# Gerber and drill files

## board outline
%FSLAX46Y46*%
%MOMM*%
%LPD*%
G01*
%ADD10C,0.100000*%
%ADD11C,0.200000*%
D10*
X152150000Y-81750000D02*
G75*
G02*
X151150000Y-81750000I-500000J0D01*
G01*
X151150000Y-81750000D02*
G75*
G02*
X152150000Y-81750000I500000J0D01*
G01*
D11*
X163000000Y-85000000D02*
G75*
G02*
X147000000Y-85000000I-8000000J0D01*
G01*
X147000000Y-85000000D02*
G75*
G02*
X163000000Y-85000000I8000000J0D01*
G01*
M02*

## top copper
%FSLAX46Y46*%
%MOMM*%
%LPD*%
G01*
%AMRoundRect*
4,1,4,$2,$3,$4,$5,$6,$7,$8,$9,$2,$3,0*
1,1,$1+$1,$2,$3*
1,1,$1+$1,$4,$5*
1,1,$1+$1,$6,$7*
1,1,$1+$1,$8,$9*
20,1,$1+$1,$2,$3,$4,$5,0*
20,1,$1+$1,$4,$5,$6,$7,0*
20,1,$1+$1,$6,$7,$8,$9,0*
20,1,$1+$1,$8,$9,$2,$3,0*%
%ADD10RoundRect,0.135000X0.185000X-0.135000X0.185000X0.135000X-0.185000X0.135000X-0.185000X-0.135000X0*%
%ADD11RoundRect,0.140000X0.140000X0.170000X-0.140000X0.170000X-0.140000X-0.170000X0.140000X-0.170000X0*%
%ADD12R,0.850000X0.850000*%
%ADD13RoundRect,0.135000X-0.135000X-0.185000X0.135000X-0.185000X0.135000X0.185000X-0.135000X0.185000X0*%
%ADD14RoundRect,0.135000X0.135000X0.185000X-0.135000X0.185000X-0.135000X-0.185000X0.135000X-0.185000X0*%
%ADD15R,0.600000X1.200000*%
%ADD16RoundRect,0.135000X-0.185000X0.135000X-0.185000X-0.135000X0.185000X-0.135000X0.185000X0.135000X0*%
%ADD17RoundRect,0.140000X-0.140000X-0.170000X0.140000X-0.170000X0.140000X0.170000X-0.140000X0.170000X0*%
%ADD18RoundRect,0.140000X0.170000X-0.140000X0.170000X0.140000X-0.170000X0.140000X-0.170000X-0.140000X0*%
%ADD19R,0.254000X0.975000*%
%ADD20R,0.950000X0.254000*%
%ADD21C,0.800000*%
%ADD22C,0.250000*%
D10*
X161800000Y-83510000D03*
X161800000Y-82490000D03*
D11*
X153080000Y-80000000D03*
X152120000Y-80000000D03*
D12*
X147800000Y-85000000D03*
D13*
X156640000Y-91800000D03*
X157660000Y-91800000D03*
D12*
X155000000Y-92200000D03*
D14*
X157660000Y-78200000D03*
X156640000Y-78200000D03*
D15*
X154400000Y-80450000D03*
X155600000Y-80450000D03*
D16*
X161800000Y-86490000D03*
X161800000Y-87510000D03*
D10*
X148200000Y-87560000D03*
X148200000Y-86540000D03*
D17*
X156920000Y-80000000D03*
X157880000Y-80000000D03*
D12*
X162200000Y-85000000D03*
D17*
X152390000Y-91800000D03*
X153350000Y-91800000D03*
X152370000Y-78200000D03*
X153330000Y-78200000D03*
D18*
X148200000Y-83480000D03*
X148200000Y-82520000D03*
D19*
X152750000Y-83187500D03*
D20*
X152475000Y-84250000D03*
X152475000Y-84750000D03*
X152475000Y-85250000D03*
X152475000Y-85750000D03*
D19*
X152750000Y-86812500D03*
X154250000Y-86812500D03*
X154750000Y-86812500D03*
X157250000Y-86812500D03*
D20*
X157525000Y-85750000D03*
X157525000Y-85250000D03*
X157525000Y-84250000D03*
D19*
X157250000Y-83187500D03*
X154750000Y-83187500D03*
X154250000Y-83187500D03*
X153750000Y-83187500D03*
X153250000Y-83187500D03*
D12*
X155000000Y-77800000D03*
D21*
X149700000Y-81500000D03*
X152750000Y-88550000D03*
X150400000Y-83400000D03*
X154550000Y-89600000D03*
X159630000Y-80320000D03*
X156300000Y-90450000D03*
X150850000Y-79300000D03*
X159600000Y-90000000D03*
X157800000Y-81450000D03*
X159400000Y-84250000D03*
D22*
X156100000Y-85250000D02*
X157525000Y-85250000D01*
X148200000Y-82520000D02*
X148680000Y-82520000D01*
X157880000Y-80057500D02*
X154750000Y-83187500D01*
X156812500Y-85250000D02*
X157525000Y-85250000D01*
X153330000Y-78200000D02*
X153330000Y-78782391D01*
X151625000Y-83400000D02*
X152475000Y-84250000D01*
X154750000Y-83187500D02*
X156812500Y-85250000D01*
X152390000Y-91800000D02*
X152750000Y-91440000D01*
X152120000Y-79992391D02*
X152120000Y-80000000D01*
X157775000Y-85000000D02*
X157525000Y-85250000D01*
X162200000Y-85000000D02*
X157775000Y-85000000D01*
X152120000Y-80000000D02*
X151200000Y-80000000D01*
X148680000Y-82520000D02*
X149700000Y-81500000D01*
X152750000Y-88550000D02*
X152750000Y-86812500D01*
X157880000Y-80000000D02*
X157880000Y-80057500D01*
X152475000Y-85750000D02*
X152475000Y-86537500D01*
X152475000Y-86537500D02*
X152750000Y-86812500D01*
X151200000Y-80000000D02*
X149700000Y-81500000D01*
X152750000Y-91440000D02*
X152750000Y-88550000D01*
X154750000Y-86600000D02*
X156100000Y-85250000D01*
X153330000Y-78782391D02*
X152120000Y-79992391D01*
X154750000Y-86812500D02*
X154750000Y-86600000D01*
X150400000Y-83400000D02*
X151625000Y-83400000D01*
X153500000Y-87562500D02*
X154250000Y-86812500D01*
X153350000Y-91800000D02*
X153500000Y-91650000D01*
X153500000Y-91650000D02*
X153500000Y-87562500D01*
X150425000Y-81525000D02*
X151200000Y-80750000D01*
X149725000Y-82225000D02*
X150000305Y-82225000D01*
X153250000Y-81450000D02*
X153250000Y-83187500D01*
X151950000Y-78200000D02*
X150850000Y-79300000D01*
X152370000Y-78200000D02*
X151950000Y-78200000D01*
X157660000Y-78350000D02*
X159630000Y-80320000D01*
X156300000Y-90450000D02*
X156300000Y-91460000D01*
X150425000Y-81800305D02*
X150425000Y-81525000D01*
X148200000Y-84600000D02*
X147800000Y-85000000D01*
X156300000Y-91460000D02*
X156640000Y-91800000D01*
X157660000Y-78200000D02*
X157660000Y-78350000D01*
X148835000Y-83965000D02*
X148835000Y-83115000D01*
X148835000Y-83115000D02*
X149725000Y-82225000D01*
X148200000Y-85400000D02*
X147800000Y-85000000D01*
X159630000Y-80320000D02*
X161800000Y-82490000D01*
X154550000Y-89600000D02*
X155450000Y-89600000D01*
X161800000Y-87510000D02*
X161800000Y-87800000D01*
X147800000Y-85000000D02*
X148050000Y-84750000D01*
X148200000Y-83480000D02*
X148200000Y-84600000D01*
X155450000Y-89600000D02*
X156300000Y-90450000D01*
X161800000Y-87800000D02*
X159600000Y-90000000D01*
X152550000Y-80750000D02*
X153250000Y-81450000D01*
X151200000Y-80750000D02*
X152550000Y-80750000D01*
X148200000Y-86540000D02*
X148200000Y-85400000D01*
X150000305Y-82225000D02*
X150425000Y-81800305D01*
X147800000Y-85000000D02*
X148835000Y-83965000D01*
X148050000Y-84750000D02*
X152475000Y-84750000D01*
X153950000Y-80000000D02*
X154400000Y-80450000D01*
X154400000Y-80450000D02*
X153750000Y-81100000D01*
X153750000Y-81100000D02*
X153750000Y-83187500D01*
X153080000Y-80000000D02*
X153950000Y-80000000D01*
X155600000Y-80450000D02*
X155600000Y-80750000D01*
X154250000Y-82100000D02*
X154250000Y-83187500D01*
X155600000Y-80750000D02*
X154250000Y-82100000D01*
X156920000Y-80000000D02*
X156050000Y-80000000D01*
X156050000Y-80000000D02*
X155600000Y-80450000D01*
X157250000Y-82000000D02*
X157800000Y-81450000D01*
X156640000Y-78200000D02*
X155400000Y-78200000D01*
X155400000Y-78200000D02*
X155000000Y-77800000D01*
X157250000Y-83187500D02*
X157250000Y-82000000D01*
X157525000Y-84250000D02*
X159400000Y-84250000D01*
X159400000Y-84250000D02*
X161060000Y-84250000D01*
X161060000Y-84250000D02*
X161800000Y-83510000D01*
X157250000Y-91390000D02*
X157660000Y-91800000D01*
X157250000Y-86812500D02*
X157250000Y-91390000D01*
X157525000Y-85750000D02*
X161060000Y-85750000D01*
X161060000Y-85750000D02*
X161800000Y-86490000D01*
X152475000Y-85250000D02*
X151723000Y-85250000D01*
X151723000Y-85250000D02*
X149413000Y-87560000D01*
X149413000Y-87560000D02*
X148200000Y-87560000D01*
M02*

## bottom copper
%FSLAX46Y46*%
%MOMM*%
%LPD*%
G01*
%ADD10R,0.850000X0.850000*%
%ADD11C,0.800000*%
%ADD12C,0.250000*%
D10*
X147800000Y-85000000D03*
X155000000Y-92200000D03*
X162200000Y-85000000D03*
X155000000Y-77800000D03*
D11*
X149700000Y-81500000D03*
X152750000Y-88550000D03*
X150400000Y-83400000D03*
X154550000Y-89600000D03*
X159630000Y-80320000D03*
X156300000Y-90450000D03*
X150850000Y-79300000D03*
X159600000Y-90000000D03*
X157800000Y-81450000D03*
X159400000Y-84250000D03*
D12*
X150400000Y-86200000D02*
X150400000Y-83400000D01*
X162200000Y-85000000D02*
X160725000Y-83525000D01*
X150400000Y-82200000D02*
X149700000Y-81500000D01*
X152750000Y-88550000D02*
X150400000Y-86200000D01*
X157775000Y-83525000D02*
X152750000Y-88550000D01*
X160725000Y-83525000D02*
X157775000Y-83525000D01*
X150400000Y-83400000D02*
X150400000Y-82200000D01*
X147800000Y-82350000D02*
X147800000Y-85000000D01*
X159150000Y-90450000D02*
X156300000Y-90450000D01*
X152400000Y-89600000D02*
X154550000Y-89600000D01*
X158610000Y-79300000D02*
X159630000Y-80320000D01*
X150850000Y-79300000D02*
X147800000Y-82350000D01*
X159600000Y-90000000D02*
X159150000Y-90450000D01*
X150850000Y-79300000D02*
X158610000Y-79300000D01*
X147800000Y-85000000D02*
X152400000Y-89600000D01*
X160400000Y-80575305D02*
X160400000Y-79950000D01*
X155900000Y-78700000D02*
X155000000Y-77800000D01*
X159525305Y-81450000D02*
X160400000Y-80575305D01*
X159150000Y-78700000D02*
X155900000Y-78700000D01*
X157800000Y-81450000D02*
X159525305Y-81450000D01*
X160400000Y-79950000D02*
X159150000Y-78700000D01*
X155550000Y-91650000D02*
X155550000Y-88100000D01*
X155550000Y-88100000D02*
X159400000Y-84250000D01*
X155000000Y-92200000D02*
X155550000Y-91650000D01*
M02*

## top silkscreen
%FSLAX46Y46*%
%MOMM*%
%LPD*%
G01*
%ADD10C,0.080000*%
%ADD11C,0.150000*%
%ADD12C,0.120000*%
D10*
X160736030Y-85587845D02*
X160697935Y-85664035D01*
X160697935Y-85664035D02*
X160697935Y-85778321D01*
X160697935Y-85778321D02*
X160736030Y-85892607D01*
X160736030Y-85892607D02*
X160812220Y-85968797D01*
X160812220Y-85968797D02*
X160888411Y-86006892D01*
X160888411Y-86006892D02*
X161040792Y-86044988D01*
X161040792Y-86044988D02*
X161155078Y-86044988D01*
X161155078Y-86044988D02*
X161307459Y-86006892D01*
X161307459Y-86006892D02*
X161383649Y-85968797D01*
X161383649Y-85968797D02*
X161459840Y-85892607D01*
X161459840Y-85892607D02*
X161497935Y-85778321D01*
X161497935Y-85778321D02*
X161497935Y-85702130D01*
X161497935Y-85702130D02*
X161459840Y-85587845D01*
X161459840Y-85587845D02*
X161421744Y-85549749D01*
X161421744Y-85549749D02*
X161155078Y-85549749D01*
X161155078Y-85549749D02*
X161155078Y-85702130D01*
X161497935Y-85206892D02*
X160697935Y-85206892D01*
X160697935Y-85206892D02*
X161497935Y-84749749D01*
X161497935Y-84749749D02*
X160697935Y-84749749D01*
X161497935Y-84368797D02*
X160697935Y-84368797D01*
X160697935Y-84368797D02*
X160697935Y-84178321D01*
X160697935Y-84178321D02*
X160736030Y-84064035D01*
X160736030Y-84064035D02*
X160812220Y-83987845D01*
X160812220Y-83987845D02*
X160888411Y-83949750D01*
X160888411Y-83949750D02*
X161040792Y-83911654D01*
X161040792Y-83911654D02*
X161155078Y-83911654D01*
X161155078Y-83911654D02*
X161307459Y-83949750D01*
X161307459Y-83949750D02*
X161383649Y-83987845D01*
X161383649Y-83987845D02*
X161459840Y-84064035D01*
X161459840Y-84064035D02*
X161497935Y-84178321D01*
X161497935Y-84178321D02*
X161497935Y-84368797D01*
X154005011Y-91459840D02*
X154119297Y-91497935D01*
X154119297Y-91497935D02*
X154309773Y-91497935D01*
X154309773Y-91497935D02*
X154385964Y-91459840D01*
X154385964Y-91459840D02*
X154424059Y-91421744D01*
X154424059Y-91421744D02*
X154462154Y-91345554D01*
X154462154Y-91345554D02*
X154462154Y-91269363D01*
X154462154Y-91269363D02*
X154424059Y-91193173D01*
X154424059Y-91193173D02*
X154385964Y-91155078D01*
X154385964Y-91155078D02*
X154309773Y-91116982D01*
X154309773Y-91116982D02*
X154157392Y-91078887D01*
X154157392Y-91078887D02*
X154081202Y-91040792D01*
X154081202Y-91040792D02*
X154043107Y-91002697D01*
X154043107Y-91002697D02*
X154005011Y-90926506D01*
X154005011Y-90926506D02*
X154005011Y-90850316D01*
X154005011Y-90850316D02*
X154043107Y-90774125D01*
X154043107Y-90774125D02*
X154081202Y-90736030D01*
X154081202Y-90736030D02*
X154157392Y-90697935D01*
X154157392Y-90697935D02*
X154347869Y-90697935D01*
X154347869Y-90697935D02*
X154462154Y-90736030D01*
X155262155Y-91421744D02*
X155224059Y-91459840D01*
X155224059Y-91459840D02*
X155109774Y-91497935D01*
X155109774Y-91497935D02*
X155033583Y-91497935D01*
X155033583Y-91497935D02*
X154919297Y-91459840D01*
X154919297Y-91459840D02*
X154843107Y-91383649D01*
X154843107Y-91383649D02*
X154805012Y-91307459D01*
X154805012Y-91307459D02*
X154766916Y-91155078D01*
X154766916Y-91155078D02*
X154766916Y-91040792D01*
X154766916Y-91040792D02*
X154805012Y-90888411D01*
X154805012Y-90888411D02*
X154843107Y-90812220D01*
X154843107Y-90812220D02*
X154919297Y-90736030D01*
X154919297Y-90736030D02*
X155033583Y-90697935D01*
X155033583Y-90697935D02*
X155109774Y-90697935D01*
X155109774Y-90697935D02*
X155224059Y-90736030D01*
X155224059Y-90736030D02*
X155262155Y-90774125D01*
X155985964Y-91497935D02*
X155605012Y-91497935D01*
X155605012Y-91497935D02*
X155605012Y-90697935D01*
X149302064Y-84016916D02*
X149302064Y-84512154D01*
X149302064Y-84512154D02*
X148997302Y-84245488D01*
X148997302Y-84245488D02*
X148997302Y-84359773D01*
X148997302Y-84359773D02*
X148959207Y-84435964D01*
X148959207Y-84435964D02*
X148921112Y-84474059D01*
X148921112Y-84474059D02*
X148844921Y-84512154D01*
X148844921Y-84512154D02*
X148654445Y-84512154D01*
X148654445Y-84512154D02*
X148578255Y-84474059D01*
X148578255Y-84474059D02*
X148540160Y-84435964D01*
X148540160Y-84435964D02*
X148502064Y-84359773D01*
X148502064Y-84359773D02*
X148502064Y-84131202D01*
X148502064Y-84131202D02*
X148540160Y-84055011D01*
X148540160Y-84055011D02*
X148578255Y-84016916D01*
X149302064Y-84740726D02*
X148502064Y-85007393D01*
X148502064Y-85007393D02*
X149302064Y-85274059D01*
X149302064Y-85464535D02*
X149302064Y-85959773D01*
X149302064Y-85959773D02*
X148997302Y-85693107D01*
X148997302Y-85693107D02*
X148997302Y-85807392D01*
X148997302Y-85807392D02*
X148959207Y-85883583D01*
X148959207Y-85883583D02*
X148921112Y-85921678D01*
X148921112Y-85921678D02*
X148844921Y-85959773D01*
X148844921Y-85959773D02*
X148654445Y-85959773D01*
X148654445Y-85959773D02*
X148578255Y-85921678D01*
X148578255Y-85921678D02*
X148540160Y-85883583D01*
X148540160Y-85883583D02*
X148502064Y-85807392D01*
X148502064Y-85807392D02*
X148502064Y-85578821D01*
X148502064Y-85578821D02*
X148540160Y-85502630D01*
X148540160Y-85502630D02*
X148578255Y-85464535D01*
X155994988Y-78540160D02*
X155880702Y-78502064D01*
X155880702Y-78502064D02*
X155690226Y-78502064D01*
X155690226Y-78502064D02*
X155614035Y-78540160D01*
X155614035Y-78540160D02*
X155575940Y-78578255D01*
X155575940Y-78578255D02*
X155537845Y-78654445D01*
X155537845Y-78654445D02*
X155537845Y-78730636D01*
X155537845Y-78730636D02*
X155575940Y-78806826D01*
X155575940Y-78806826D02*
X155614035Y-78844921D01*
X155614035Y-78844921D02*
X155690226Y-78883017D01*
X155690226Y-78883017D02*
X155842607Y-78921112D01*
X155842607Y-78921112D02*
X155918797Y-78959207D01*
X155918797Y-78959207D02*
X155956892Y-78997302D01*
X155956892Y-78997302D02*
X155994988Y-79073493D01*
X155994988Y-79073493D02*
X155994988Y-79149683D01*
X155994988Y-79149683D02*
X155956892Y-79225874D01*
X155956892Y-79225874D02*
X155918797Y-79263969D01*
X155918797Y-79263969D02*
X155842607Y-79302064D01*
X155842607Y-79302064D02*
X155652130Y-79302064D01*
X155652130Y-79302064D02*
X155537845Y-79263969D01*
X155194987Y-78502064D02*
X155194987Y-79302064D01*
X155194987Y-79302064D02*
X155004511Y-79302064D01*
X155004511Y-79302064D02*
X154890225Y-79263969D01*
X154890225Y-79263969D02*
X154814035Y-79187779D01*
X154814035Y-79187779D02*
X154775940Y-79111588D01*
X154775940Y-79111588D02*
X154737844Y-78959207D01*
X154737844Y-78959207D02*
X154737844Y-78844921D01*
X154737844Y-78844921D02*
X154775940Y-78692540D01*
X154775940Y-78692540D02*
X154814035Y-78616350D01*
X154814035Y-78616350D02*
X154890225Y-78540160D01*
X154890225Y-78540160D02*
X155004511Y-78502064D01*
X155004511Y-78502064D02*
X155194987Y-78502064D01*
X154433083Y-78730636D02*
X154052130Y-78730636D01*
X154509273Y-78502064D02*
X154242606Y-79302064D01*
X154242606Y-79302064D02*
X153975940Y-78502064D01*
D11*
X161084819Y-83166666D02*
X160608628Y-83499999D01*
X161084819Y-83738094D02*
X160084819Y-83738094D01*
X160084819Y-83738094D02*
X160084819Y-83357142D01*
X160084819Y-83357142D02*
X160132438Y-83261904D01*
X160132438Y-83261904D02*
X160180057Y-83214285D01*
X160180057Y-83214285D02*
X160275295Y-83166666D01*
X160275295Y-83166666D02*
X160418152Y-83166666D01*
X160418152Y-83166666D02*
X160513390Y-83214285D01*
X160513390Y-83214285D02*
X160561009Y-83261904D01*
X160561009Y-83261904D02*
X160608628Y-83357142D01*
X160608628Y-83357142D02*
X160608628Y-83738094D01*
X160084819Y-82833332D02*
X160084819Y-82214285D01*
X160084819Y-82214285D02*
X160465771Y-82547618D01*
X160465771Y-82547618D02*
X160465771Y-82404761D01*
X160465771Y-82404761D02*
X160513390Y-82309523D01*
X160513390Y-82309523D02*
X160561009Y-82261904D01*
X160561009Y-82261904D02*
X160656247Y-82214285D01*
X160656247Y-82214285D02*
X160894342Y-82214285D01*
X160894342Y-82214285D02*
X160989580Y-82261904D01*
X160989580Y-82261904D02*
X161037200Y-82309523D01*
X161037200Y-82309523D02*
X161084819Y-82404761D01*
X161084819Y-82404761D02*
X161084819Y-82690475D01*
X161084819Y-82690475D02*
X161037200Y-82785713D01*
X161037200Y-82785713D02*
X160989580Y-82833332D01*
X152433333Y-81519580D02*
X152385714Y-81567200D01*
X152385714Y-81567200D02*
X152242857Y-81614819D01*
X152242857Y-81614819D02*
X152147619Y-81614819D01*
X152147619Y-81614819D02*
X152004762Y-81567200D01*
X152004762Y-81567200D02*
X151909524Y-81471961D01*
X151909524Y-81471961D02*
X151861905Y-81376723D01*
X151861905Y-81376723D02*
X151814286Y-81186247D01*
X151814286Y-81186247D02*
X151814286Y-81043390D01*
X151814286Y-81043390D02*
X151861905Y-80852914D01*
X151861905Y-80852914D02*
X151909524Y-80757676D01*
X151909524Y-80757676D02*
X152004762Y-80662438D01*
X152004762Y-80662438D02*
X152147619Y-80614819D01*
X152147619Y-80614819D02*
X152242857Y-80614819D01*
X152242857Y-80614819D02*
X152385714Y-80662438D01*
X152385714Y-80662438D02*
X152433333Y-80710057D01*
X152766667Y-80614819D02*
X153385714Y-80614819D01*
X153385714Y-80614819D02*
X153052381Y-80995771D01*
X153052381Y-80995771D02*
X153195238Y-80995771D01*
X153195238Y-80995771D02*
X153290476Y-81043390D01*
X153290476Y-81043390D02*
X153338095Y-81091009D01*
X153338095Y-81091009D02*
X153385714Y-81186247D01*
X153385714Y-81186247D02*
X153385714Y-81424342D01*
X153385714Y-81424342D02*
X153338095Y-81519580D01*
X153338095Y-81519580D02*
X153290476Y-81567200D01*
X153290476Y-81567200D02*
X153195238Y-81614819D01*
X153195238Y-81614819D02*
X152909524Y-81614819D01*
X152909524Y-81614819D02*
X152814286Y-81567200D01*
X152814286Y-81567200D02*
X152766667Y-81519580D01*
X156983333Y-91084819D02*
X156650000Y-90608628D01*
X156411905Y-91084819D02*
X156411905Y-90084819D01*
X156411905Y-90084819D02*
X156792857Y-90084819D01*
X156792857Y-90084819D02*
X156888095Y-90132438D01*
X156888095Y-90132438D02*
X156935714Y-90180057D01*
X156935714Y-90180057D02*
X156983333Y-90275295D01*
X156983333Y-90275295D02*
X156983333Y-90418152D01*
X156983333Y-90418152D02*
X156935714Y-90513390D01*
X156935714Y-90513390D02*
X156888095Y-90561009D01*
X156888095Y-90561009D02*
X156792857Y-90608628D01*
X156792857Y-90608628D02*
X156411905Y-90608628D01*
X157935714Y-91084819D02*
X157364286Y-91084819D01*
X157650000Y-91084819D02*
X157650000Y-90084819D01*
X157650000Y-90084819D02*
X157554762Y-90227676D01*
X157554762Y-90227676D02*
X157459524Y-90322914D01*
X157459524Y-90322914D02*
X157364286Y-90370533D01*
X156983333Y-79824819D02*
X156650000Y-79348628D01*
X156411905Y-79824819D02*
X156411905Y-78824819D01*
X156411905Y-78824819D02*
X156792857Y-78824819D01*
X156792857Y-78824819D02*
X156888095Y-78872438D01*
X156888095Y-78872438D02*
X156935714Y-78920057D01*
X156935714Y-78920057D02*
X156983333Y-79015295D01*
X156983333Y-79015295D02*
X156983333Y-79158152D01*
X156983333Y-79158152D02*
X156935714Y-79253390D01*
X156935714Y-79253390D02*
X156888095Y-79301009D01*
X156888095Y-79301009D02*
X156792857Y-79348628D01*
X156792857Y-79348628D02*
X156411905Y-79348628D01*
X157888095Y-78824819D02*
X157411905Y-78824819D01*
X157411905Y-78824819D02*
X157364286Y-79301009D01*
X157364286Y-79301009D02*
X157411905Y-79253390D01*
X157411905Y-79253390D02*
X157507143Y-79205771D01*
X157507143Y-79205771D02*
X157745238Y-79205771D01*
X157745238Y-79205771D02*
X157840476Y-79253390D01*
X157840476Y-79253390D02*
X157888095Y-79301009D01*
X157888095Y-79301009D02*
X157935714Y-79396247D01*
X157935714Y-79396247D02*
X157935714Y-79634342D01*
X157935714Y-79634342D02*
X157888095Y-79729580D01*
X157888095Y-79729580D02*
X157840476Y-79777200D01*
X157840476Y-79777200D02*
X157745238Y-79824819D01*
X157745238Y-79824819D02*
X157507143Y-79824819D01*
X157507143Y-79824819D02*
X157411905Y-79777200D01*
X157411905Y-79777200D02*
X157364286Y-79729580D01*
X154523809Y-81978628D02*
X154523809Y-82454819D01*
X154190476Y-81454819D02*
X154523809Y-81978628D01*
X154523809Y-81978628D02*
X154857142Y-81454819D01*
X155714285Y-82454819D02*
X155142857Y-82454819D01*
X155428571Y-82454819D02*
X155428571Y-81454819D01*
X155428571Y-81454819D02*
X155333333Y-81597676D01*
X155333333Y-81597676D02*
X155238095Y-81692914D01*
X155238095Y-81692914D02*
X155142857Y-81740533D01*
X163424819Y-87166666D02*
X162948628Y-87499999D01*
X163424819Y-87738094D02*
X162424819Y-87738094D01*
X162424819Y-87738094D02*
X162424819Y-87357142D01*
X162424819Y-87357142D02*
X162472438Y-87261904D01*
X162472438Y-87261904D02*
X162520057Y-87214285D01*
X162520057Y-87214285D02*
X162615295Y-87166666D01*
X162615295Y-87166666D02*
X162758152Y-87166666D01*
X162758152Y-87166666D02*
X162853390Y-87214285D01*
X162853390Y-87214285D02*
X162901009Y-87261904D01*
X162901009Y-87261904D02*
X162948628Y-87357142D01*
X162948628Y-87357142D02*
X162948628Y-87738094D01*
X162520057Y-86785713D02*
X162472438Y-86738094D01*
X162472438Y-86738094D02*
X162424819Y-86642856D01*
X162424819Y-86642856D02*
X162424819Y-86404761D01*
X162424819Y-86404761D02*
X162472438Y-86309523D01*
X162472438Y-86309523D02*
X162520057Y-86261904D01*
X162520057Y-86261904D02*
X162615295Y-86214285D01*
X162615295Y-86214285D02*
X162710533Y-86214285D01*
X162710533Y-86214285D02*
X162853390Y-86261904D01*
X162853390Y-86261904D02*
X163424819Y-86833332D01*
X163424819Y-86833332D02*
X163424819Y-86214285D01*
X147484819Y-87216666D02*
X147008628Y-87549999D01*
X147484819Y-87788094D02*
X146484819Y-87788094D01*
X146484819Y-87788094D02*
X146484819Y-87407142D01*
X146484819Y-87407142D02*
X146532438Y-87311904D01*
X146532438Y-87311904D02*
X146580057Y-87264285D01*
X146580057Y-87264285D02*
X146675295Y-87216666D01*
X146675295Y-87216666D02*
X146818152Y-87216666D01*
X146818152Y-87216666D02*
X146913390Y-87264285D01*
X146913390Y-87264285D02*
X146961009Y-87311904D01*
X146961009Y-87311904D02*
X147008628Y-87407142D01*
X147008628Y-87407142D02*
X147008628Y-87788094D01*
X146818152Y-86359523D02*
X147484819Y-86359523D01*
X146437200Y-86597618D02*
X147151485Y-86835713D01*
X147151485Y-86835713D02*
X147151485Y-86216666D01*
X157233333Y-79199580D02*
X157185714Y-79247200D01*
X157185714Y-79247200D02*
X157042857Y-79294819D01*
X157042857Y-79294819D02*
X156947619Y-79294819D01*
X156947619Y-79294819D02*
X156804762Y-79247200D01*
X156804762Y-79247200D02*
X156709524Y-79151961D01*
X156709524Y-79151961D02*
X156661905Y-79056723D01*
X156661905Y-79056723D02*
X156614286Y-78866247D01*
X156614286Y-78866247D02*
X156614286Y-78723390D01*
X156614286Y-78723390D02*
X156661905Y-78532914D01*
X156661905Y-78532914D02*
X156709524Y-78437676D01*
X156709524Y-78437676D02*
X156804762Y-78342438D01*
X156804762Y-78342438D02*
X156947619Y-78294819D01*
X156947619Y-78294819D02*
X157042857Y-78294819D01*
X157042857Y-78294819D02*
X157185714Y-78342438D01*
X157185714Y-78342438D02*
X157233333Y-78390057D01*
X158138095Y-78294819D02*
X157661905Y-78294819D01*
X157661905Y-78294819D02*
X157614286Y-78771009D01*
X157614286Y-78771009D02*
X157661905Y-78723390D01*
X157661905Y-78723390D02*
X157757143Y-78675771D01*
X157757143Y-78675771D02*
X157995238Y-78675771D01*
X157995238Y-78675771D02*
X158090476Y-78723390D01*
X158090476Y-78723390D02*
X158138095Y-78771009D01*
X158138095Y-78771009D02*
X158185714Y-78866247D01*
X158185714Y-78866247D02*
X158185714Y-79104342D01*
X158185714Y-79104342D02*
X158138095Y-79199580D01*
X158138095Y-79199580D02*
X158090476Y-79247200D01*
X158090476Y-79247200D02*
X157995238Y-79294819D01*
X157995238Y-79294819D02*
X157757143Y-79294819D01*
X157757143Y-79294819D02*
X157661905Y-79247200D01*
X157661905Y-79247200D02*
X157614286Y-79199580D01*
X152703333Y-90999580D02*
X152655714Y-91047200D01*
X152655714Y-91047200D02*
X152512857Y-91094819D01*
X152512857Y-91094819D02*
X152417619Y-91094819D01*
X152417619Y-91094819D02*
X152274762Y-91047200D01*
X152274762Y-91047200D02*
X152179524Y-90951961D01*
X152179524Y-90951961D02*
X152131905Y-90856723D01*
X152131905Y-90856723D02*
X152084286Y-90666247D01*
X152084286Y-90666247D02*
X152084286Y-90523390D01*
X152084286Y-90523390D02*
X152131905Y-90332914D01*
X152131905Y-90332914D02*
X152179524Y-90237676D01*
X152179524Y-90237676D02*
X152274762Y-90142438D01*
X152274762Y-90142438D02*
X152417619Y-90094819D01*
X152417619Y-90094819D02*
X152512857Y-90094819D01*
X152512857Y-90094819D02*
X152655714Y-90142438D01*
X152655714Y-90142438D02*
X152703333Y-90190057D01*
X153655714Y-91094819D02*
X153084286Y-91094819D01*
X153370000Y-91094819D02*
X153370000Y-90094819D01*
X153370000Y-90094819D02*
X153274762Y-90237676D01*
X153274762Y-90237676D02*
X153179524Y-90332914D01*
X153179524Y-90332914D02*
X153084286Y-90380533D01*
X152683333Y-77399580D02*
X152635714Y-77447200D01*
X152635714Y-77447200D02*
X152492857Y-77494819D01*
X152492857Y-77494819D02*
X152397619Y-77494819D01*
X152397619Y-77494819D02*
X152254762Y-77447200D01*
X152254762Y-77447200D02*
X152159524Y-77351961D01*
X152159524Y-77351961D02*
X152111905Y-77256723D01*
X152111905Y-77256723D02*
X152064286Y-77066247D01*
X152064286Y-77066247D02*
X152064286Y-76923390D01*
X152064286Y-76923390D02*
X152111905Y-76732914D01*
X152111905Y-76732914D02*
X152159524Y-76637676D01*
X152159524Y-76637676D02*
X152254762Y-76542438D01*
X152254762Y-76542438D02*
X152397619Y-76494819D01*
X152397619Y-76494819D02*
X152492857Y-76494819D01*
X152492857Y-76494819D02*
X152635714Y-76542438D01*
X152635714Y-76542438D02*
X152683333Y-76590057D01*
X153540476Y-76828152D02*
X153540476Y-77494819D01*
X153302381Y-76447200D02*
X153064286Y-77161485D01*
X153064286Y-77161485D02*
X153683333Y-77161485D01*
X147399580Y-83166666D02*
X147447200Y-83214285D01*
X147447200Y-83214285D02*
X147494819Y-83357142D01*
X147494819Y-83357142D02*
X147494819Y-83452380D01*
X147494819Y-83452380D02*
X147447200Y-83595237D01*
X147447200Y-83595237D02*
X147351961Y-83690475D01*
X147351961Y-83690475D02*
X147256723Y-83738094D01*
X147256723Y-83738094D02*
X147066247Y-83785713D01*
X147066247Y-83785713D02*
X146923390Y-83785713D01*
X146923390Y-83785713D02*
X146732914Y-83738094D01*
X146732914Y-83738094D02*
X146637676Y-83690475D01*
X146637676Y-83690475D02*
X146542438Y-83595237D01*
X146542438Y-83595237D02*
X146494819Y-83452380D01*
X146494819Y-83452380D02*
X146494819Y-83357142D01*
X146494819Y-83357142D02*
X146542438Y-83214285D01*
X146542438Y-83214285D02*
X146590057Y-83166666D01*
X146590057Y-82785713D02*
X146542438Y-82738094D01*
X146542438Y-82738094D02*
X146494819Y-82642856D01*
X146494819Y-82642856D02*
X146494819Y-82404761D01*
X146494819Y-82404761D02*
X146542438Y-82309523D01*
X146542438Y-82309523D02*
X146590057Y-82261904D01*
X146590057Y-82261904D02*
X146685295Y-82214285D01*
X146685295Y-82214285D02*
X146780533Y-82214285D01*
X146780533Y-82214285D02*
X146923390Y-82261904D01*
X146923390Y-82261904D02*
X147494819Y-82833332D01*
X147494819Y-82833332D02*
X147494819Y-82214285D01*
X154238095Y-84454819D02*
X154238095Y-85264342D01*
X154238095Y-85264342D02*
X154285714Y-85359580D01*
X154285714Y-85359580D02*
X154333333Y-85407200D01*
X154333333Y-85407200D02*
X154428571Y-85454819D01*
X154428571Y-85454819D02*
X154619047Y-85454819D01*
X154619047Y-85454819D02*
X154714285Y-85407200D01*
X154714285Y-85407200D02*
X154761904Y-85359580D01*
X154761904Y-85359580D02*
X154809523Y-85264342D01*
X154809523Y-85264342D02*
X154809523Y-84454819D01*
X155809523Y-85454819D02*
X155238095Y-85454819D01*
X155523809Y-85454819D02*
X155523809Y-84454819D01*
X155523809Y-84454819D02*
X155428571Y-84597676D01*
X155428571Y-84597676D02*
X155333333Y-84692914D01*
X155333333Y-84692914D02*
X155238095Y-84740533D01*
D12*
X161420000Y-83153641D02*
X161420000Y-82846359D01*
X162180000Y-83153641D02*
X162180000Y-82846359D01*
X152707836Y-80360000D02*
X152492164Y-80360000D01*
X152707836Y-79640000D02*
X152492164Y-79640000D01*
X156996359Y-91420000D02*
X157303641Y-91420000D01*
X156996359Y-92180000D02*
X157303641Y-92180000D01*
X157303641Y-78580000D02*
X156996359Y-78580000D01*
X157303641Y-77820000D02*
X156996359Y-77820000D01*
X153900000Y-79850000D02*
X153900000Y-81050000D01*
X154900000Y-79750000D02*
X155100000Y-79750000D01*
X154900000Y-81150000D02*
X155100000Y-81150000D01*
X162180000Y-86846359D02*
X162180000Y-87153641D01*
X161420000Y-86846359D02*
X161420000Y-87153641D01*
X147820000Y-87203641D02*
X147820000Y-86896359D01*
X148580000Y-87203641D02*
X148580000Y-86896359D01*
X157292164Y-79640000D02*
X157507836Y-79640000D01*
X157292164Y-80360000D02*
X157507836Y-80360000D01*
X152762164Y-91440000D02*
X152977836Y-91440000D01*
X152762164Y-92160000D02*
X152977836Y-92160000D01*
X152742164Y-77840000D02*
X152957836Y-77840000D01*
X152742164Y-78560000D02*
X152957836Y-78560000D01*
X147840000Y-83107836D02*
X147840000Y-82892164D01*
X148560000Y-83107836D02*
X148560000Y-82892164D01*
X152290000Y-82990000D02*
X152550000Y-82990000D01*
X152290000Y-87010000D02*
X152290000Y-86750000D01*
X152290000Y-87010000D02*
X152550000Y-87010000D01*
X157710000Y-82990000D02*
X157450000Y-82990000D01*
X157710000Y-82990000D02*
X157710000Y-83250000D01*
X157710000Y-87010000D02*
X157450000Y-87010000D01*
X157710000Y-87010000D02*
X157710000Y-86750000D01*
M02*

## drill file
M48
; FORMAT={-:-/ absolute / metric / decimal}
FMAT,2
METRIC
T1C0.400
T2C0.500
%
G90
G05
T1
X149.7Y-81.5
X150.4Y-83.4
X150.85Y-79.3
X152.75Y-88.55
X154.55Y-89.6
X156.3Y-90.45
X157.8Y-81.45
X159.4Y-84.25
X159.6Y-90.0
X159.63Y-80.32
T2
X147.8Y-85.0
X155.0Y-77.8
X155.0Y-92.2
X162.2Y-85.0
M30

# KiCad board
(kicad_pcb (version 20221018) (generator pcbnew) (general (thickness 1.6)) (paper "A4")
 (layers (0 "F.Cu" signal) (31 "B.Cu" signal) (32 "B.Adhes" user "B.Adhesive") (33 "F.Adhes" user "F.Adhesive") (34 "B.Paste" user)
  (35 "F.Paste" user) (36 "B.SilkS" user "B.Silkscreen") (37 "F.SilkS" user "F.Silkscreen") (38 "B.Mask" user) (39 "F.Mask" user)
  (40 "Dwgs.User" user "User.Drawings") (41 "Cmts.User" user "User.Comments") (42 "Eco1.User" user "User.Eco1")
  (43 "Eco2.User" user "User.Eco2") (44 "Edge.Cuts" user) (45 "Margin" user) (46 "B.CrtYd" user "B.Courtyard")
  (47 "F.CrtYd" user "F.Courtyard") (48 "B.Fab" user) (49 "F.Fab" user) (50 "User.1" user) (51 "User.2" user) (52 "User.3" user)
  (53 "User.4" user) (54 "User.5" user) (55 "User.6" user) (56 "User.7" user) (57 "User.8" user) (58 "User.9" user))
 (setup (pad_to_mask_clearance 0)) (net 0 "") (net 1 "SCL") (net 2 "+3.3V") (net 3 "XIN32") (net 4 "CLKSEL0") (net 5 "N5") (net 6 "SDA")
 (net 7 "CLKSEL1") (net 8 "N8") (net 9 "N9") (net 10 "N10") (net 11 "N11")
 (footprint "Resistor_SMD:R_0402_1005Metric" (layer "F.Cu") (at 161.8 83 90)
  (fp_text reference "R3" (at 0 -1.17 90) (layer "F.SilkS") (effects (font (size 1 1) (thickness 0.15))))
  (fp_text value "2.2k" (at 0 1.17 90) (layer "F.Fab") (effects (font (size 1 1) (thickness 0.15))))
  (fp_line (start -0.153641 -0.38) (end 0.153641 -0.38) (stroke (width 0.12) (type solid)) (layer "F.SilkS"))
  (fp_line (start -0.153641 0.38) (end 0.153641 0.38) (stroke (width 0.12) (type solid)) (layer "F.SilkS"))
  (pad "1" smd roundrect (at -0.51 0 90) (size 0.54 0.64) (layers "F.Cu" "F.Paste" "F.Mask") (roundrect_rratio 0.25) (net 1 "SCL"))
  (pad "2" smd roundrect (at 0.51 0 90) (size 0.54 0.64) (layers "F.Cu" "F.Paste" "F.Mask") (roundrect_rratio 0.25) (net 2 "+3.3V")))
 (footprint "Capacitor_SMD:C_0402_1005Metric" (layer "F.Cu") (at 152.6 80 180)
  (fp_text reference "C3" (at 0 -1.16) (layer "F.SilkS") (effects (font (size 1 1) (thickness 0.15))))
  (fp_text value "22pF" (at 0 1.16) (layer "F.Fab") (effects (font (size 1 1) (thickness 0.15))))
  (fp_line (start -0.107836 -0.36) (end 0.107836 -0.36) (stroke (width 0.12) (type solid)) (layer "F.SilkS"))
  (fp_line (start -0.107836 0.36) (end 0.107836 0.36) (stroke (width 0.12) (type solid)) (layer "F.SilkS"))
  (pad "1" smd roundrect (at -0.48 0 180) (size 0.56 0.62) (layers "F.Cu" "F.Paste" "F.Mask") (roundrect_rratio 0.25) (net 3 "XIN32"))
  (pad "2" smd roundrect (at 0.48 0 180) (size 0.56 0.62) (layers "F.Cu" "F.Paste" "F.Mask") (roundrect_rratio 0.25) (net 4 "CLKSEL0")))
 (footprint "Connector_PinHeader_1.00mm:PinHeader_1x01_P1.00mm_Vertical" (layer "F.Cu") (at 147.8 85)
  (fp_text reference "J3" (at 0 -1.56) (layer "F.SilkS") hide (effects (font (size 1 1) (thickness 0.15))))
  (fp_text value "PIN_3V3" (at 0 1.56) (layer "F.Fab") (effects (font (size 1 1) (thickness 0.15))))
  (pad "1" thru_hole rect (at 0 0) (size 0.85 0.85) (drill 0.5) (layers "*.Cu" "*.Mask") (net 2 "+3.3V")))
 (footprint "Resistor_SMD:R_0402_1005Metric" (layer "F.Cu") (at 157.15 91.8)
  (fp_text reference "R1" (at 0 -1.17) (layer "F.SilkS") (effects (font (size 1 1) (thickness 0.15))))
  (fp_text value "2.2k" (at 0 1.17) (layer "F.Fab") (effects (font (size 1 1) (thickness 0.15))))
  (fp_line (start -0.153641 -0.38) (end 0.153641 -0.38) (stroke (width 0.12) (type solid)) (layer "F.SilkS"))
  (fp_line (start -0.153641 0.38) (end 0.153641 0.38) (stroke (width 0.12) (type solid)) (layer "F.SilkS"))
  (pad "1" smd roundrect (at -0.51 0) (size 0.54 0.64) (layers "F.Cu" "F.Paste" "F.Mask") (roundrect_rratio 0.25) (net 2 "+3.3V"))
  (pad "2" smd roundrect (at 0.51 0) (size 0.54 0.64) (layers "F.Cu" "F.Paste" "F.Mask") (roundrect_rratio 0.25) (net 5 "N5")))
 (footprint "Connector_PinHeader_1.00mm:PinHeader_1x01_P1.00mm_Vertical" (layer "F.Cu") (at 155 92.2)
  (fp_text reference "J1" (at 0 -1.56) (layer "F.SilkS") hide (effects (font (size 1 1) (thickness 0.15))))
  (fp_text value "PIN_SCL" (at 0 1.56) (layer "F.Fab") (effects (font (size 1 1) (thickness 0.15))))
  (pad "1" thru_hole rect (at 0 0) (size 0.85 0.85) (drill 0.5) (layers "*.Cu" "*.Mask") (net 1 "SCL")))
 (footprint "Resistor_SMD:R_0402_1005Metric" (layer "F.Cu") (at 157.15 78.2 180)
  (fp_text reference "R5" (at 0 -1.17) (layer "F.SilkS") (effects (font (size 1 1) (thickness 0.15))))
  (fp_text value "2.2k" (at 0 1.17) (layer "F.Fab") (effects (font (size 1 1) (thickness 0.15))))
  (fp_line (start -0.153641 -0.38) (end 0.153641 -0.38) (stroke (width 0.12) (type solid)) (layer "F.SilkS"))
  (fp_line (start -0.153641 0.38) (end 0.153641 0.38) (stroke (width 0.12) (type solid)) (layer "F.SilkS"))
  (pad "1" smd roundrect (at -0.51 0 180) (size 0.54 0.64) (layers "F.Cu" "F.Paste" "F.Mask") (roundrect_rratio 0.25) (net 2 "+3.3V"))
  (pad "2" smd roundrect (at 0.51 0 180) (size 0.54 0.64) (layers "F.Cu" "F.Paste" "F.Mask") (roundrect_rratio 0.25) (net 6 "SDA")))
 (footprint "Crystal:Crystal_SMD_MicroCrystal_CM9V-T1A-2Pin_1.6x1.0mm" (layer "F.Cu") (at 155 80.45)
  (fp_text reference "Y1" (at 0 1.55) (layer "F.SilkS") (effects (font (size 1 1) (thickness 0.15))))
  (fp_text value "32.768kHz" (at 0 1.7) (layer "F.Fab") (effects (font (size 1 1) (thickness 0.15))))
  (fp_line (start -1.1 -0.6) (end -1.1 0.6) (stroke (width 0.12) (type solid)) (layer "F.SilkS"))
  (fp_line (start -0.1 -0.7) (end 0.1 -0.7) (stroke (width 0.12) (type solid)) (layer "F.SilkS"))
  (fp_line (start -0.1 0.7) (end 0.1 0.7) (stroke (width 0.12) (type solid)) (layer "F.SilkS"))
  (pad "1" smd rect (at -0.6 0) (size 0.6 1.2) (layers "F.Cu" "F.Paste" "F.Mask") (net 3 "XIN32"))
  (pad "2" smd rect (at 0.6 0) (size 0.6 1.2) (layers "F.Cu" "F.Paste" "F.Mask") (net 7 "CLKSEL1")))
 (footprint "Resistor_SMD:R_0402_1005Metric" (layer "F.Cu") (at 161.8 87 -90)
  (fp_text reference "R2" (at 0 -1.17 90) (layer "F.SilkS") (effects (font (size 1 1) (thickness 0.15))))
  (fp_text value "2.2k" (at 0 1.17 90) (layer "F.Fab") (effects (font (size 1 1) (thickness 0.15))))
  (fp_line (start -0.153641 -0.38) (end 0.153641 -0.38) (stroke (width 0.12) (type solid)) (layer "F.SilkS"))
  (fp_line (start -0.153641 0.38) (end 0.153641 0.38) (stroke (width 0.12) (type solid)) (layer "F.SilkS"))
  (pad "1" smd roundrect (at -0.51 0 270) (size 0.54 0.64) (layers "F.Cu" "F.Paste" "F.Mask") (roundrect_rratio 0.25) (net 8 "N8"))
  (pad "2" smd roundrect (at 0.51 0 270) (size 0.54 0.64) (layers "F.Cu" "F.Paste" "F.Mask") (roundrect_rratio 0.25) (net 2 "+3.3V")))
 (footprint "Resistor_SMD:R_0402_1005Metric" (layer "F.Cu") (at 148.2 87.05 90)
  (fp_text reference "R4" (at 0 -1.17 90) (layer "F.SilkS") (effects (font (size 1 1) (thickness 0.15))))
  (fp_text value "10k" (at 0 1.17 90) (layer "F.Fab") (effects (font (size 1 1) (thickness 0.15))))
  (fp_line (start -0.153641 -0.38) (end 0.153641 -0.38) (stroke (width 0.12) (type solid)) (layer "F.SilkS"))
  (fp_line (start -0.153641 0.38) (end 0.153641 0.38) (stroke (width 0.12) (type solid)) (layer "F.SilkS"))
  (pad "1" smd roundrect (at -0.51 0 90) (size 0.54 0.64) (layers "F.Cu" "F.Paste" "F.Mask") (roundrect_rratio 0.25) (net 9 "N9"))
  (pad "2" smd roundrect (at 0.51 0 90) (size 0.54 0.64) (layers "F.Cu" "F.Paste" "F.Mask") (roundrect_rratio 0.25) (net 2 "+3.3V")))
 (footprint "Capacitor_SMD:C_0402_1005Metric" (layer "F.Cu") (at 157.4 80)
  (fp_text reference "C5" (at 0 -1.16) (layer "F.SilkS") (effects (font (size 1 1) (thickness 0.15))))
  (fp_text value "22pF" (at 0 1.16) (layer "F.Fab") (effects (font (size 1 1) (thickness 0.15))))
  (fp_line (start -0.107836 -0.36) (end 0.107836 -0.36) (stroke (width 0.12) (type solid)) (layer "F.SilkS"))
  (fp_line (start -0.107836 0.36) (end 0.107836 0.36) (stroke (width 0.12) (type solid)) (layer "F.SilkS"))
  (pad "1" smd roundrect (at -0.48 0) (size 0.56 0.62) (layers "F.Cu" "F.Paste" "F.Mask") (roundrect_rratio 0.25) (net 7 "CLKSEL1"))
  (pad "2" smd roundrect (at 0.48 0) (size 0.56 0.62) (layers "F.Cu" "F.Paste" "F.Mask") (roundrect_rratio 0.25) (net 4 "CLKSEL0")))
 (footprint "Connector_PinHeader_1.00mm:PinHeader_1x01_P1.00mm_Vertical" (layer "F.Cu") (at 162.2 85)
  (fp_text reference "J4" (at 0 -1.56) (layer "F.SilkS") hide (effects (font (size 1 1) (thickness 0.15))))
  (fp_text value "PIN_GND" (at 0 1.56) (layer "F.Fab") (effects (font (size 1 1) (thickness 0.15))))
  (pad "1" thru_hole rect (at 0 0) (size 0.85 0.85) (drill 0.5) (layers "*.Cu" "*.Mask") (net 4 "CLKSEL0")))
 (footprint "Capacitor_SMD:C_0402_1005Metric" (layer "F.Cu") (at 152.87 91.8)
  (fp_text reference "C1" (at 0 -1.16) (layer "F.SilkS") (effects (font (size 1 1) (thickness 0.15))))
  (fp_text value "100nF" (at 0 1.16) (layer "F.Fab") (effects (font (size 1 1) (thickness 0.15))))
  (fp_line (start -0.107836 -0.36) (end 0.107836 -0.36) (stroke (width 0.12) (type solid)) (layer "F.SilkS"))
  (fp_line (start -0.107836 0.36) (end 0.107836 0.36) (stroke (width 0.12) (type solid)) (layer "F.SilkS"))
  (pad "1" smd roundrect (at -0.48 0) (size 0.56 0.62) (layers "F.Cu" "F.Paste" "F.Mask") (roundrect_rratio 0.25) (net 4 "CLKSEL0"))
  (pad "2" smd roundrect (at 0.48 0) (size 0.56 0.62) (layers "F.Cu" "F.Paste" "F.Mask") (roundrect_rratio 0.25) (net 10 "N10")))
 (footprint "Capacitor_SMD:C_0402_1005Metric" (layer "F.Cu") (at 152.85 78.2)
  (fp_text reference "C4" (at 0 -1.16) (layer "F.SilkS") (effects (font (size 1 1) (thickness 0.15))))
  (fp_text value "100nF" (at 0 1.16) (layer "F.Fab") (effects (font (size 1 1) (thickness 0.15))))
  (fp_line (start -0.107836 -0.36) (end 0.107836 -0.36) (stroke (width 0.12) (type solid)) (layer "F.SilkS"))
  (fp_line (start -0.107836 0.36) (end 0.107836 0.36) (stroke (width 0.12) (type solid)) (layer "F.SilkS"))
  (pad "1" smd roundrect (at -0.48 0) (size 0.56 0.62) (layers "F.Cu" "F.Paste" "F.Mask") (roundrect_rratio 0.25) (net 2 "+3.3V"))
  (pad "2" smd roundrect (at 0.48 0) (size 0.56 0.62) (layers "F.Cu" "F.Paste" "F.Mask") (roundrect_rratio 0.25) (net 4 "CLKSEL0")))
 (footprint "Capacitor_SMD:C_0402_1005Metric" (layer "F.Cu") (at 148.2 83 90)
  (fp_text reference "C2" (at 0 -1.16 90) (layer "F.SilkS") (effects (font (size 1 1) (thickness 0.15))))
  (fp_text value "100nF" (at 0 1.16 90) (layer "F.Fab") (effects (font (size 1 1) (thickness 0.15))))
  (fp_line (start -0.107836 -0.36) (end 0.107836 -0.36) (stroke (width 0.12) (type solid)) (layer "F.SilkS"))
  (fp_line (start -0.107836 0.36) (end 0.107836 0.36) (stroke (width 0.12) (type solid)) (layer "F.SilkS"))
  (pad "1" smd roundrect (at -0.48 0 90) (size 0.56 0.62) (layers "F.Cu" "F.Paste" "F.Mask") (roundrect_rratio 0.25) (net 2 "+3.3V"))
  (pad "2" smd roundrect (at 0.48 0 90) (size 0.56 0.62) (layers "F.Cu" "F.Paste" "F.Mask") (roundrect_rratio 0.25) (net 4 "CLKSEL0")))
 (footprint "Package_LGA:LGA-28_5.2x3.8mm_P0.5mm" (layer "F.Cu") (at 155 85)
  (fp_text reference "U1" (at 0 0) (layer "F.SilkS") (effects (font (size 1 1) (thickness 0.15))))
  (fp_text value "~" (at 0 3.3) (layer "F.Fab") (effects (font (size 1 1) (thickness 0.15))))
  (fp_line (start -2.71 -2.01) (end -2.45 -2.01) (stroke (width 0.12) (type solid)) (layer "F.SilkS"))
  (fp_line (start -2.71 2.01) (end -2.71 1.75) (stroke (width 0.12) (type solid)) (layer "F.SilkS"))
  (fp_line (start -2.71 2.01) (end -2.45 2.01) (stroke (width 0.12) (type solid)) (layer "F.SilkS"))
  (fp_line (start 2.71 -2.01) (end 2.45 -2.01) (stroke (width 0.12) (type solid)) (layer "F.SilkS"))
  (fp_line (start 2.71 -2.01) (end 2.71 -1.75) (stroke (width 0.12) (type solid)) (layer "F.SilkS"))
  (fp_line (start 2.71 2.01) (end 2.45 2.01) (stroke (width 0.12) (type solid)) (layer "F.SilkS"))
  (fp_line (start 2.71 2.01) (end 2.71 1.75) (stroke (width 0.12) (type solid)) (layer "F.SilkS"))
  (pad "1" smd rect (at -2.25 -1.8125) (size 0.254 0.975) (layers "F.Cu" "F.Paste" "F.Mask") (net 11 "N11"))
  (pad "2" smd rect (at -2.525 -0.75 90) (size 0.254 0.95) (layers "F.Cu" "F.Paste" "F.Mask") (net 4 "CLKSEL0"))
  (pad "3" smd rect (at -2.525 -0.25 90) (size 0.254 0.95) (layers "F.Cu" "F.Paste" "F.Mask") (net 2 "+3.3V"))
  (pad "4" smd rect (at -2.525 0.25 90) (size 0.254 0.95) (layers "F.Cu" "F.Paste" "F.Mask") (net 9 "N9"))
  (pad "5" smd rect (at -2.525 0.75 90) (size 0.254 0.95) (layers "F.Cu" "F.Paste" "F.Mask") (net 4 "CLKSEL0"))
  (pad "6" smd rect (at -2.25 1.8125) (size 0.254 0.975) (layers "F.Cu" "F.Paste" "F.Mask") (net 4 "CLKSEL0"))
  (pad "9" smd rect (at -0.75 1.8125) (size 0.254 0.975) (layers "F.Cu" "F.Paste" "F.Mask") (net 10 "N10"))
  (pad "10" smd rect (at -0.25 1.8125) (size 0.254 0.975) (layers "F.Cu" "F.Paste" "F.Mask") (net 4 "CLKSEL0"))
  (pad "15" smd rect (at 2.25 1.8125) (size 0.254 0.975) (layers "F.Cu" "F.Paste" "F.Mask") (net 5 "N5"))
  (pad "16" smd rect (at 2.525 0.75 90) (size 0.254 0.95) (layers "F.Cu" "F.Paste" "F.Mask") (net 8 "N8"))
  (pad "17" smd rect (at 2.525 0.25 90) (size 0.254 0.95) (layers "F.Cu" "F.Paste" "F.Mask") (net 4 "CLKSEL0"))
  (pad "19" smd rect (at 2.525 -0.75 90) (size 0.254 0.95) (layers "F.Cu" "F.Paste" "F.Mask") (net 1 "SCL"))
  (pad "20" smd rect (at 2.25 -1.8125) (size 0.254 0.975) (layers "F.Cu" "F.Paste" "F.Mask") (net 6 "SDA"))
  (pad "25" smd rect (at -0.25 -1.8125) (size 0.254 0.975) (layers "F.Cu" "F.Paste" "F.Mask") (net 4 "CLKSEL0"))
  (pad "26" smd rect (at -0.75 -1.8125) (size 0.254 0.975) (layers "F.Cu" "F.Paste" "F.Mask") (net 7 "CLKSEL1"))
  (pad "27" smd rect (at -1.25 -1.8125) (size 0.254 0.975) (layers "F.Cu" "F.Paste" "F.Mask") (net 3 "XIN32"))
  (pad "28" smd rect (at -1.75 -1.8125) (size 0.254 0.975) (layers "F.Cu" "F.Paste" "F.Mask") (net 2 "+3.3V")))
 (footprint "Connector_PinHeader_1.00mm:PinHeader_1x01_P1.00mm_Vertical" (layer "F.Cu") (at 155 77.8)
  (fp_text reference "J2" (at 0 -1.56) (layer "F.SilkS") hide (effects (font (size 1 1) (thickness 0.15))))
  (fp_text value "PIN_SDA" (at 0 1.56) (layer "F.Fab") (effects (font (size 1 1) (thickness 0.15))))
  (pad "1" thru_hole rect (at 0 0) (size 0.85 0.85) (drill 0.5) (layers "*.Cu" "*.Mask") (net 6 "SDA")))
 (gr_circle (center 151.65 81.75) (end 152.15 81.75) (stroke (width 0.1) (type default)) (fill none) (layer "Edge.Cuts"))
 (gr_circle (center 155 85) (end 163 85) (stroke (width 0.2) (type default)) (fill none) (layer "Edge.Cuts"))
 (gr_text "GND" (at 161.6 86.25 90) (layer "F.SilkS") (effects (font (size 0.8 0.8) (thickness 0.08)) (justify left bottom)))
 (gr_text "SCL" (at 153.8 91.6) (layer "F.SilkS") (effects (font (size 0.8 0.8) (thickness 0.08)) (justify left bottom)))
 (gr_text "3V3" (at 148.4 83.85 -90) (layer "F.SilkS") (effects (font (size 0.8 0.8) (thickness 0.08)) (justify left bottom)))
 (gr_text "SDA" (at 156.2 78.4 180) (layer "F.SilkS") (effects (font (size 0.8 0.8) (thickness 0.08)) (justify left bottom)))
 (segment (start 156.1 85.25) (end 157.525 85.25) (width 0.25) (layer "F.Cu") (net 4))
 (segment (start 148.2 82.52) (end 148.68 82.52) (width 0.25) (layer "F.Cu") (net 4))
 (segment (start 157.88 80.0575) (end 154.75 83.1875) (width 0.25) (layer "F.Cu") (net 4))
 (segment (start 156.8125 85.25) (end 157.525 85.25) (width 0.25) (layer "F.Cu") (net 4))
 (segment (start 153.33 78.2) (end 153.33 78.782391) (width 0.25) (layer "F.Cu") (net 4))
 (segment (start 151.625 83.4) (end 152.475 84.25) (width 0.25) (layer "F.Cu") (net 4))
 (segment (start 154.75 83.1875) (end 156.8125 85.25) (width 0.25) (layer "F.Cu") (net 4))
 (segment (start 152.39 91.8) (end 152.75 91.44) (width 0.25) (layer "F.Cu") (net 4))
 (segment (start 152.12 79.992391) (end 152.12 80) (width 0.25) (layer "F.Cu") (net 4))
 (segment (start 157.775 85) (end 157.525 85.25) (width 0.25) (layer "F.Cu") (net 4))
 (segment (start 162.2 85) (end 157.775 85) (width 0.25) (layer "F.Cu") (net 4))
 (segment (start 152.12 80) (end 151.2 80) (width 0.25) (layer "F.Cu") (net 4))
 (segment (start 148.68 82.52) (end 149.7 81.5) (width 0.25) (layer "F.Cu") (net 4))
 (segment (start 152.75 88.55) (end 152.75 86.8125) (width 0.25) (layer "F.Cu") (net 4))
 (segment (start 157.88 80) (end 157.88 80.0575) (width 0.25) (layer "F.Cu") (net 4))
 (segment (start 152.475 85.75) (end 152.475 86.5375) (width 0.25) (layer "F.Cu") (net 4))
 (segment (start 152.475 86.5375) (end 152.75 86.8125) (width 0.25) (layer "F.Cu") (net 4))
 (segment (start 151.2 80) (end 149.7 81.5) (width 0.25) (layer "F.Cu") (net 4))
 (segment (start 152.75 91.44) (end 152.75 88.55) (width 0.25) (layer "F.Cu") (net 4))
 (segment (start 154.75 86.6) (end 156.1 85.25) (width 0.25) (layer "F.Cu") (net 4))
 (segment (start 153.33 78.782391) (end 152.12 79.992391) (width 0.25) (layer "F.Cu") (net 4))
 (segment (start 154.75 86.8125) (end 154.75 86.6) (width 0.25) (layer "F.Cu") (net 4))
 (segment (start 150.4 83.4) (end 151.625 83.4) (width 0.25) (layer "F.Cu") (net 4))
 (via (at 149.7 81.5) (size 0.8) (drill 0.4) (layers "F.Cu" "B.Cu") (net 4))
 (via (at 152.75 88.55) (size 0.8) (drill 0.4) (layers "F.Cu" "B.Cu") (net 4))
 (via (at 150.4 83.4) (size 0.8) (drill 0.4) (layers "F.Cu" "B.Cu") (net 4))
 (segment (start 150.4 86.2) (end 150.4 83.4) (width 0.25) (layer "B.Cu") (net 4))
 (segment (start 162.2 85) (end 160.725 83.525) (width 0.25) (layer "B.Cu") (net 4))
 (segment (start 150.4 82.2) (end 149.7 81.5) (width 0.25) (layer "B.Cu") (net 4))
 (segment (start 152.75 88.55) (end 150.4 86.2) (width 0.25) (layer "B.Cu") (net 4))
 (segment (start 157.775 83.525) (end 152.75 88.55) (width 0.25) (layer "B.Cu") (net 4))
 (segment (start 160.725 83.525) (end 157.775 83.525) (width 0.25) (layer "B.Cu") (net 4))
 (segment (start 150.4 83.4) (end 150.4 82.2) (width 0.25) (layer "B.Cu") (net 4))
 (segment (start 153.5 87.5625) (end 154.25 86.8125) (width 0.25) (layer "F.Cu") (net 10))
 (segment (start 153.35 91.8) (end 153.5 91.65) (width 0.25) (layer "F.Cu") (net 10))
 (segment (start 153.5 91.65) (end 153.5 87.5625) (width 0.25) (layer "F.Cu") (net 10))
 (segment (start 150.425 81.525) (end 151.2 80.75) (width 0.25) (layer "F.Cu") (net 2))
 (segment (start 149.725 82.225) (end 150.000305 82.225) (width 0.25) (layer "F.Cu") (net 2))
 (segment (start 153.25 81.45) (end 153.25 83.1875) (width 0.25) (layer "F.Cu") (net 2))
 (segment (start 151.95 78.2) (end 150.85 79.3) (width 0.25) (layer "F.Cu") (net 2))
 (segment (start 152.37 78.2) (end 151.95 78.2) (width 0.25) (layer "F.Cu") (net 2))
 (segment (start 157.66 78.35) (end 159.63 80.32) (width 0.25) (layer "F.Cu") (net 2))
 (segment (start 156.3 90.45) (end 156.3 91.46) (width 0.25) (layer "F.Cu") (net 2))
 (segment (start 150.425 81.800305) (end 150.425 81.525) (width 0.25) (layer "F.Cu") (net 2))
 (segment (start 148.2 84.6) (end 147.8 85) (width 0.25) (layer "F.Cu") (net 2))
 (segment (start 156.3 91.46) (end 156.64 91.8) (width 0.25) (layer "F.Cu") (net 2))
 (segment (start 157.66 78.2) (end 157.66 78.35) (width 0.25) (layer "F.Cu") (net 2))
 (segment (start 148.835 83.965) (end 148.835 83.115) (width 0.25) (layer "F.Cu") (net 2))
 (segment (start 148.835 83.115) (end 149.725 82.225) (width 0.25) (layer "F.Cu") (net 2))
 (segment (start 148.2 85.4) (end 147.8 85) (width 0.25) (layer "F.Cu") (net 2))
 (segment (start 159.63 80.32) (end 161.8 82.49) (width 0.25) (layer "F.Cu") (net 2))
 (segment (start 154.55 89.6) (end 155.45 89.6) (width 0.25) (layer "F.Cu") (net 2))
 (segment (start 161.8 87.51) (end 161.8 87.8) (width 0.25) (layer "F.Cu") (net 2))
 (segment (start 147.8 85) (end 148.05 84.75) (width 0.25) (layer "F.Cu") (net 2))
 (segment (start 148.2 83.48) (end 148.2 84.6) (width 0.25) (layer "F.Cu") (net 2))
 (segment (start 155.45 89.6) (end 156.3 90.45) (width 0.25) (layer "F.Cu") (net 2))
 (segment (start 161.8 87.8) (end 159.6 90) (width 0.25) (layer "F.Cu") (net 2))
 (segment (start 152.55 80.75) (end 153.25 81.45) (width 0.25) (layer "F.Cu") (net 2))
 (segment (start 151.2 80.75) (end 152.55 80.75) (width 0.25) (layer "F.Cu") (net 2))
 (segment (start 148.2 86.54) (end 148.2 85.4) (width 0.25) (layer "F.Cu") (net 2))
 (segment (start 150.000305 82.225) (end 150.425 81.800305) (width 0.25) (layer "F.Cu") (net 2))
 (segment (start 147.8 85) (end 148.835 83.965) (width 0.25) (layer "F.Cu") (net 2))
 (segment (start 148.05 84.75) (end 152.475 84.75) (width 0.25) (layer "F.Cu") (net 2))
 (via (at 154.55 89.6) (size 0.8) (drill 0.4) (layers "F.Cu" "B.Cu") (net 2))
 (via (at 159.63 80.32) (size 0.8) (drill 0.4) (layers "F.Cu" "B.Cu") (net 2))
 (via (at 156.3 90.45) (size 0.8) (drill 0.4) (layers "F.Cu" "B.Cu") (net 2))
 (via (at 150.85 79.3) (size 0.8) (drill 0.4) (layers "F.Cu" "B.Cu") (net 2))
 (via (at 159.6 90) (size 0.8) (drill 0.4) (layers "F.Cu" "B.Cu") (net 2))
 (segment (start 147.8 82.35) (end 147.8 85) (width 0.25) (layer "B.Cu") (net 2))
 (segment (start 159.15 90.45) (end 156.3 90.45) (width 0.25) (layer "B.Cu") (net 2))
 (segment (start 152.4 89.6) (end 154.55 89.6) (width 0.25) (layer "B.Cu") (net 2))
 (segment (start 158.61 79.3) (end 159.63 80.32) (width 0.25) (layer "B.Cu") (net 2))
 (segment (start 150.85 79.3) (end 147.8 82.35) (width 0.25) (layer "B.Cu") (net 2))
 (segment (start 159.6 90) (end 159.15 90.45) (width 0.25) (layer "B.Cu") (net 2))
 (segment (start 150.85 79.3) (end 158.61 79.3) (width 0.25) (layer "B.Cu") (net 2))
 (segment (start 147.8 85) (end 152.4 89.6) (width 0.25) (layer "B.Cu") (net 2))
 (segment (start 153.95 80) (end 154.4 80.45) (width 0.25) (layer "F.Cu") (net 3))
 (segment (start 154.4 80.45) (end 153.75 81.1) (width 0.25) (layer "F.Cu") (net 3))
 (segment (start 153.75 81.1) (end 153.75 83.1875) (width 0.25) (layer "F.Cu") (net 3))
 (segment (start 153.08 80) (end 153.95 80) (width 0.25) (layer "F.Cu") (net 3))
 (segment (start 155.6 80.45) (end 155.6 80.75) (width 0.25) (layer "F.Cu") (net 7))
 (segment (start 154.25 82.1) (end 154.25 83.1875) (width 0.25) (layer "F.Cu") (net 7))
 (segment (start 155.6 80.75) (end 154.25 82.1) (width 0.25) (layer "F.Cu") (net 7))
 (segment (start 156.92 80) (end 156.05 80) (width 0.25) (layer "F.Cu") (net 7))
 (segment (start 156.05 80) (end 155.6 80.45) (width 0.25) (layer "F.Cu") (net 7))
 (segment (start 157.25 82) (end 157.8 81.45) (width 0.25) (layer "F.Cu") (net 6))
 (segment (start 156.64 78.2) (end 155.4 78.2) (width 0.25) (layer "F.Cu") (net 6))
 (segment (start 155.4 78.2) (end 155 77.8) (width 0.25) (layer "F.Cu") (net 6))
 (segment (start 157.25 83.1875) (end 157.25 82) (width 0.25) (layer "F.Cu") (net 6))
 (via (at 157.8 81.45) (size 0.8) (drill 0.4) (layers "F.Cu" "B.Cu") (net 6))
 (segment (start 160.4 80.575305) (end 160.4 79.95) (width 0.25) (layer "B.Cu") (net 6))
 (segment (start 155.9 78.7) (end 155 77.8) (width 0.25) (layer "B.Cu") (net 6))
 (segment (start 159.525305 81.45) (end 160.4 80.575305) (width 0.25) (layer "B.Cu") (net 6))
 (segment (start 159.15 78.7) (end 155.9 78.7) (width 0.25) (layer "B.Cu") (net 6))
 (segment (start 157.8 81.45) (end 159.525305 81.45) (width 0.25) (layer "B.Cu") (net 6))
 (segment (start 160.4 79.95) (end 159.15 78.7) (width 0.25) (layer "B.Cu") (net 6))
 (segment (start 157.525 84.25) (end 159.4 84.25) (width 0.25) (layer "F.Cu") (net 1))
 (segment (start 159.4 84.25) (end 161.06 84.25) (width 0.25) (layer "F.Cu") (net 1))
 (segment (start 161.06 84.25) (end 161.8 83.51) (width 0.25) (layer "F.Cu") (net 1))
 (via (at 159.4 84.25) (size 0.8) (drill 0.4) (layers "F.Cu" "B.Cu") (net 1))
 (segment (start 155.55 91.65) (end 155.55 88.1) (width 0.25) (layer "B.Cu") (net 1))
 (segment (start 155.55 88.1) (end 159.4 84.25) (width 0.25) (layer "B.Cu") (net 1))
 (segment (start 155 92.2) (end 155.55 91.65) (width 0.25) (layer "B.Cu") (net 1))
 (segment (start 157.25 91.39) (end 157.66 91.8) (width 0.25) (layer "F.Cu") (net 5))
 (segment (start 157.25 86.8125) (end 157.25 91.39) (width 0.25) (layer "F.Cu") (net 5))
 (segment (start 157.525 85.75) (end 161.06 85.75) (width 0.25) (layer "F.Cu") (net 8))
 (segment (start 161.06 85.75) (end 161.8 86.49) (width 0.25) (layer "F.Cu") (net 8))
 (segment (start 152.475 85.25) (end 151.723 85.25) (width 0.25) (layer "F.Cu") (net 9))
 (segment (start 151.723 85.25) (end 149.413 87.56) (width 0.25) (layer "F.Cu") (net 9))
 (segment (start 149.413 87.56) (end 148.2 87.56) (width 0.25) (layer "F.Cu") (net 9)))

